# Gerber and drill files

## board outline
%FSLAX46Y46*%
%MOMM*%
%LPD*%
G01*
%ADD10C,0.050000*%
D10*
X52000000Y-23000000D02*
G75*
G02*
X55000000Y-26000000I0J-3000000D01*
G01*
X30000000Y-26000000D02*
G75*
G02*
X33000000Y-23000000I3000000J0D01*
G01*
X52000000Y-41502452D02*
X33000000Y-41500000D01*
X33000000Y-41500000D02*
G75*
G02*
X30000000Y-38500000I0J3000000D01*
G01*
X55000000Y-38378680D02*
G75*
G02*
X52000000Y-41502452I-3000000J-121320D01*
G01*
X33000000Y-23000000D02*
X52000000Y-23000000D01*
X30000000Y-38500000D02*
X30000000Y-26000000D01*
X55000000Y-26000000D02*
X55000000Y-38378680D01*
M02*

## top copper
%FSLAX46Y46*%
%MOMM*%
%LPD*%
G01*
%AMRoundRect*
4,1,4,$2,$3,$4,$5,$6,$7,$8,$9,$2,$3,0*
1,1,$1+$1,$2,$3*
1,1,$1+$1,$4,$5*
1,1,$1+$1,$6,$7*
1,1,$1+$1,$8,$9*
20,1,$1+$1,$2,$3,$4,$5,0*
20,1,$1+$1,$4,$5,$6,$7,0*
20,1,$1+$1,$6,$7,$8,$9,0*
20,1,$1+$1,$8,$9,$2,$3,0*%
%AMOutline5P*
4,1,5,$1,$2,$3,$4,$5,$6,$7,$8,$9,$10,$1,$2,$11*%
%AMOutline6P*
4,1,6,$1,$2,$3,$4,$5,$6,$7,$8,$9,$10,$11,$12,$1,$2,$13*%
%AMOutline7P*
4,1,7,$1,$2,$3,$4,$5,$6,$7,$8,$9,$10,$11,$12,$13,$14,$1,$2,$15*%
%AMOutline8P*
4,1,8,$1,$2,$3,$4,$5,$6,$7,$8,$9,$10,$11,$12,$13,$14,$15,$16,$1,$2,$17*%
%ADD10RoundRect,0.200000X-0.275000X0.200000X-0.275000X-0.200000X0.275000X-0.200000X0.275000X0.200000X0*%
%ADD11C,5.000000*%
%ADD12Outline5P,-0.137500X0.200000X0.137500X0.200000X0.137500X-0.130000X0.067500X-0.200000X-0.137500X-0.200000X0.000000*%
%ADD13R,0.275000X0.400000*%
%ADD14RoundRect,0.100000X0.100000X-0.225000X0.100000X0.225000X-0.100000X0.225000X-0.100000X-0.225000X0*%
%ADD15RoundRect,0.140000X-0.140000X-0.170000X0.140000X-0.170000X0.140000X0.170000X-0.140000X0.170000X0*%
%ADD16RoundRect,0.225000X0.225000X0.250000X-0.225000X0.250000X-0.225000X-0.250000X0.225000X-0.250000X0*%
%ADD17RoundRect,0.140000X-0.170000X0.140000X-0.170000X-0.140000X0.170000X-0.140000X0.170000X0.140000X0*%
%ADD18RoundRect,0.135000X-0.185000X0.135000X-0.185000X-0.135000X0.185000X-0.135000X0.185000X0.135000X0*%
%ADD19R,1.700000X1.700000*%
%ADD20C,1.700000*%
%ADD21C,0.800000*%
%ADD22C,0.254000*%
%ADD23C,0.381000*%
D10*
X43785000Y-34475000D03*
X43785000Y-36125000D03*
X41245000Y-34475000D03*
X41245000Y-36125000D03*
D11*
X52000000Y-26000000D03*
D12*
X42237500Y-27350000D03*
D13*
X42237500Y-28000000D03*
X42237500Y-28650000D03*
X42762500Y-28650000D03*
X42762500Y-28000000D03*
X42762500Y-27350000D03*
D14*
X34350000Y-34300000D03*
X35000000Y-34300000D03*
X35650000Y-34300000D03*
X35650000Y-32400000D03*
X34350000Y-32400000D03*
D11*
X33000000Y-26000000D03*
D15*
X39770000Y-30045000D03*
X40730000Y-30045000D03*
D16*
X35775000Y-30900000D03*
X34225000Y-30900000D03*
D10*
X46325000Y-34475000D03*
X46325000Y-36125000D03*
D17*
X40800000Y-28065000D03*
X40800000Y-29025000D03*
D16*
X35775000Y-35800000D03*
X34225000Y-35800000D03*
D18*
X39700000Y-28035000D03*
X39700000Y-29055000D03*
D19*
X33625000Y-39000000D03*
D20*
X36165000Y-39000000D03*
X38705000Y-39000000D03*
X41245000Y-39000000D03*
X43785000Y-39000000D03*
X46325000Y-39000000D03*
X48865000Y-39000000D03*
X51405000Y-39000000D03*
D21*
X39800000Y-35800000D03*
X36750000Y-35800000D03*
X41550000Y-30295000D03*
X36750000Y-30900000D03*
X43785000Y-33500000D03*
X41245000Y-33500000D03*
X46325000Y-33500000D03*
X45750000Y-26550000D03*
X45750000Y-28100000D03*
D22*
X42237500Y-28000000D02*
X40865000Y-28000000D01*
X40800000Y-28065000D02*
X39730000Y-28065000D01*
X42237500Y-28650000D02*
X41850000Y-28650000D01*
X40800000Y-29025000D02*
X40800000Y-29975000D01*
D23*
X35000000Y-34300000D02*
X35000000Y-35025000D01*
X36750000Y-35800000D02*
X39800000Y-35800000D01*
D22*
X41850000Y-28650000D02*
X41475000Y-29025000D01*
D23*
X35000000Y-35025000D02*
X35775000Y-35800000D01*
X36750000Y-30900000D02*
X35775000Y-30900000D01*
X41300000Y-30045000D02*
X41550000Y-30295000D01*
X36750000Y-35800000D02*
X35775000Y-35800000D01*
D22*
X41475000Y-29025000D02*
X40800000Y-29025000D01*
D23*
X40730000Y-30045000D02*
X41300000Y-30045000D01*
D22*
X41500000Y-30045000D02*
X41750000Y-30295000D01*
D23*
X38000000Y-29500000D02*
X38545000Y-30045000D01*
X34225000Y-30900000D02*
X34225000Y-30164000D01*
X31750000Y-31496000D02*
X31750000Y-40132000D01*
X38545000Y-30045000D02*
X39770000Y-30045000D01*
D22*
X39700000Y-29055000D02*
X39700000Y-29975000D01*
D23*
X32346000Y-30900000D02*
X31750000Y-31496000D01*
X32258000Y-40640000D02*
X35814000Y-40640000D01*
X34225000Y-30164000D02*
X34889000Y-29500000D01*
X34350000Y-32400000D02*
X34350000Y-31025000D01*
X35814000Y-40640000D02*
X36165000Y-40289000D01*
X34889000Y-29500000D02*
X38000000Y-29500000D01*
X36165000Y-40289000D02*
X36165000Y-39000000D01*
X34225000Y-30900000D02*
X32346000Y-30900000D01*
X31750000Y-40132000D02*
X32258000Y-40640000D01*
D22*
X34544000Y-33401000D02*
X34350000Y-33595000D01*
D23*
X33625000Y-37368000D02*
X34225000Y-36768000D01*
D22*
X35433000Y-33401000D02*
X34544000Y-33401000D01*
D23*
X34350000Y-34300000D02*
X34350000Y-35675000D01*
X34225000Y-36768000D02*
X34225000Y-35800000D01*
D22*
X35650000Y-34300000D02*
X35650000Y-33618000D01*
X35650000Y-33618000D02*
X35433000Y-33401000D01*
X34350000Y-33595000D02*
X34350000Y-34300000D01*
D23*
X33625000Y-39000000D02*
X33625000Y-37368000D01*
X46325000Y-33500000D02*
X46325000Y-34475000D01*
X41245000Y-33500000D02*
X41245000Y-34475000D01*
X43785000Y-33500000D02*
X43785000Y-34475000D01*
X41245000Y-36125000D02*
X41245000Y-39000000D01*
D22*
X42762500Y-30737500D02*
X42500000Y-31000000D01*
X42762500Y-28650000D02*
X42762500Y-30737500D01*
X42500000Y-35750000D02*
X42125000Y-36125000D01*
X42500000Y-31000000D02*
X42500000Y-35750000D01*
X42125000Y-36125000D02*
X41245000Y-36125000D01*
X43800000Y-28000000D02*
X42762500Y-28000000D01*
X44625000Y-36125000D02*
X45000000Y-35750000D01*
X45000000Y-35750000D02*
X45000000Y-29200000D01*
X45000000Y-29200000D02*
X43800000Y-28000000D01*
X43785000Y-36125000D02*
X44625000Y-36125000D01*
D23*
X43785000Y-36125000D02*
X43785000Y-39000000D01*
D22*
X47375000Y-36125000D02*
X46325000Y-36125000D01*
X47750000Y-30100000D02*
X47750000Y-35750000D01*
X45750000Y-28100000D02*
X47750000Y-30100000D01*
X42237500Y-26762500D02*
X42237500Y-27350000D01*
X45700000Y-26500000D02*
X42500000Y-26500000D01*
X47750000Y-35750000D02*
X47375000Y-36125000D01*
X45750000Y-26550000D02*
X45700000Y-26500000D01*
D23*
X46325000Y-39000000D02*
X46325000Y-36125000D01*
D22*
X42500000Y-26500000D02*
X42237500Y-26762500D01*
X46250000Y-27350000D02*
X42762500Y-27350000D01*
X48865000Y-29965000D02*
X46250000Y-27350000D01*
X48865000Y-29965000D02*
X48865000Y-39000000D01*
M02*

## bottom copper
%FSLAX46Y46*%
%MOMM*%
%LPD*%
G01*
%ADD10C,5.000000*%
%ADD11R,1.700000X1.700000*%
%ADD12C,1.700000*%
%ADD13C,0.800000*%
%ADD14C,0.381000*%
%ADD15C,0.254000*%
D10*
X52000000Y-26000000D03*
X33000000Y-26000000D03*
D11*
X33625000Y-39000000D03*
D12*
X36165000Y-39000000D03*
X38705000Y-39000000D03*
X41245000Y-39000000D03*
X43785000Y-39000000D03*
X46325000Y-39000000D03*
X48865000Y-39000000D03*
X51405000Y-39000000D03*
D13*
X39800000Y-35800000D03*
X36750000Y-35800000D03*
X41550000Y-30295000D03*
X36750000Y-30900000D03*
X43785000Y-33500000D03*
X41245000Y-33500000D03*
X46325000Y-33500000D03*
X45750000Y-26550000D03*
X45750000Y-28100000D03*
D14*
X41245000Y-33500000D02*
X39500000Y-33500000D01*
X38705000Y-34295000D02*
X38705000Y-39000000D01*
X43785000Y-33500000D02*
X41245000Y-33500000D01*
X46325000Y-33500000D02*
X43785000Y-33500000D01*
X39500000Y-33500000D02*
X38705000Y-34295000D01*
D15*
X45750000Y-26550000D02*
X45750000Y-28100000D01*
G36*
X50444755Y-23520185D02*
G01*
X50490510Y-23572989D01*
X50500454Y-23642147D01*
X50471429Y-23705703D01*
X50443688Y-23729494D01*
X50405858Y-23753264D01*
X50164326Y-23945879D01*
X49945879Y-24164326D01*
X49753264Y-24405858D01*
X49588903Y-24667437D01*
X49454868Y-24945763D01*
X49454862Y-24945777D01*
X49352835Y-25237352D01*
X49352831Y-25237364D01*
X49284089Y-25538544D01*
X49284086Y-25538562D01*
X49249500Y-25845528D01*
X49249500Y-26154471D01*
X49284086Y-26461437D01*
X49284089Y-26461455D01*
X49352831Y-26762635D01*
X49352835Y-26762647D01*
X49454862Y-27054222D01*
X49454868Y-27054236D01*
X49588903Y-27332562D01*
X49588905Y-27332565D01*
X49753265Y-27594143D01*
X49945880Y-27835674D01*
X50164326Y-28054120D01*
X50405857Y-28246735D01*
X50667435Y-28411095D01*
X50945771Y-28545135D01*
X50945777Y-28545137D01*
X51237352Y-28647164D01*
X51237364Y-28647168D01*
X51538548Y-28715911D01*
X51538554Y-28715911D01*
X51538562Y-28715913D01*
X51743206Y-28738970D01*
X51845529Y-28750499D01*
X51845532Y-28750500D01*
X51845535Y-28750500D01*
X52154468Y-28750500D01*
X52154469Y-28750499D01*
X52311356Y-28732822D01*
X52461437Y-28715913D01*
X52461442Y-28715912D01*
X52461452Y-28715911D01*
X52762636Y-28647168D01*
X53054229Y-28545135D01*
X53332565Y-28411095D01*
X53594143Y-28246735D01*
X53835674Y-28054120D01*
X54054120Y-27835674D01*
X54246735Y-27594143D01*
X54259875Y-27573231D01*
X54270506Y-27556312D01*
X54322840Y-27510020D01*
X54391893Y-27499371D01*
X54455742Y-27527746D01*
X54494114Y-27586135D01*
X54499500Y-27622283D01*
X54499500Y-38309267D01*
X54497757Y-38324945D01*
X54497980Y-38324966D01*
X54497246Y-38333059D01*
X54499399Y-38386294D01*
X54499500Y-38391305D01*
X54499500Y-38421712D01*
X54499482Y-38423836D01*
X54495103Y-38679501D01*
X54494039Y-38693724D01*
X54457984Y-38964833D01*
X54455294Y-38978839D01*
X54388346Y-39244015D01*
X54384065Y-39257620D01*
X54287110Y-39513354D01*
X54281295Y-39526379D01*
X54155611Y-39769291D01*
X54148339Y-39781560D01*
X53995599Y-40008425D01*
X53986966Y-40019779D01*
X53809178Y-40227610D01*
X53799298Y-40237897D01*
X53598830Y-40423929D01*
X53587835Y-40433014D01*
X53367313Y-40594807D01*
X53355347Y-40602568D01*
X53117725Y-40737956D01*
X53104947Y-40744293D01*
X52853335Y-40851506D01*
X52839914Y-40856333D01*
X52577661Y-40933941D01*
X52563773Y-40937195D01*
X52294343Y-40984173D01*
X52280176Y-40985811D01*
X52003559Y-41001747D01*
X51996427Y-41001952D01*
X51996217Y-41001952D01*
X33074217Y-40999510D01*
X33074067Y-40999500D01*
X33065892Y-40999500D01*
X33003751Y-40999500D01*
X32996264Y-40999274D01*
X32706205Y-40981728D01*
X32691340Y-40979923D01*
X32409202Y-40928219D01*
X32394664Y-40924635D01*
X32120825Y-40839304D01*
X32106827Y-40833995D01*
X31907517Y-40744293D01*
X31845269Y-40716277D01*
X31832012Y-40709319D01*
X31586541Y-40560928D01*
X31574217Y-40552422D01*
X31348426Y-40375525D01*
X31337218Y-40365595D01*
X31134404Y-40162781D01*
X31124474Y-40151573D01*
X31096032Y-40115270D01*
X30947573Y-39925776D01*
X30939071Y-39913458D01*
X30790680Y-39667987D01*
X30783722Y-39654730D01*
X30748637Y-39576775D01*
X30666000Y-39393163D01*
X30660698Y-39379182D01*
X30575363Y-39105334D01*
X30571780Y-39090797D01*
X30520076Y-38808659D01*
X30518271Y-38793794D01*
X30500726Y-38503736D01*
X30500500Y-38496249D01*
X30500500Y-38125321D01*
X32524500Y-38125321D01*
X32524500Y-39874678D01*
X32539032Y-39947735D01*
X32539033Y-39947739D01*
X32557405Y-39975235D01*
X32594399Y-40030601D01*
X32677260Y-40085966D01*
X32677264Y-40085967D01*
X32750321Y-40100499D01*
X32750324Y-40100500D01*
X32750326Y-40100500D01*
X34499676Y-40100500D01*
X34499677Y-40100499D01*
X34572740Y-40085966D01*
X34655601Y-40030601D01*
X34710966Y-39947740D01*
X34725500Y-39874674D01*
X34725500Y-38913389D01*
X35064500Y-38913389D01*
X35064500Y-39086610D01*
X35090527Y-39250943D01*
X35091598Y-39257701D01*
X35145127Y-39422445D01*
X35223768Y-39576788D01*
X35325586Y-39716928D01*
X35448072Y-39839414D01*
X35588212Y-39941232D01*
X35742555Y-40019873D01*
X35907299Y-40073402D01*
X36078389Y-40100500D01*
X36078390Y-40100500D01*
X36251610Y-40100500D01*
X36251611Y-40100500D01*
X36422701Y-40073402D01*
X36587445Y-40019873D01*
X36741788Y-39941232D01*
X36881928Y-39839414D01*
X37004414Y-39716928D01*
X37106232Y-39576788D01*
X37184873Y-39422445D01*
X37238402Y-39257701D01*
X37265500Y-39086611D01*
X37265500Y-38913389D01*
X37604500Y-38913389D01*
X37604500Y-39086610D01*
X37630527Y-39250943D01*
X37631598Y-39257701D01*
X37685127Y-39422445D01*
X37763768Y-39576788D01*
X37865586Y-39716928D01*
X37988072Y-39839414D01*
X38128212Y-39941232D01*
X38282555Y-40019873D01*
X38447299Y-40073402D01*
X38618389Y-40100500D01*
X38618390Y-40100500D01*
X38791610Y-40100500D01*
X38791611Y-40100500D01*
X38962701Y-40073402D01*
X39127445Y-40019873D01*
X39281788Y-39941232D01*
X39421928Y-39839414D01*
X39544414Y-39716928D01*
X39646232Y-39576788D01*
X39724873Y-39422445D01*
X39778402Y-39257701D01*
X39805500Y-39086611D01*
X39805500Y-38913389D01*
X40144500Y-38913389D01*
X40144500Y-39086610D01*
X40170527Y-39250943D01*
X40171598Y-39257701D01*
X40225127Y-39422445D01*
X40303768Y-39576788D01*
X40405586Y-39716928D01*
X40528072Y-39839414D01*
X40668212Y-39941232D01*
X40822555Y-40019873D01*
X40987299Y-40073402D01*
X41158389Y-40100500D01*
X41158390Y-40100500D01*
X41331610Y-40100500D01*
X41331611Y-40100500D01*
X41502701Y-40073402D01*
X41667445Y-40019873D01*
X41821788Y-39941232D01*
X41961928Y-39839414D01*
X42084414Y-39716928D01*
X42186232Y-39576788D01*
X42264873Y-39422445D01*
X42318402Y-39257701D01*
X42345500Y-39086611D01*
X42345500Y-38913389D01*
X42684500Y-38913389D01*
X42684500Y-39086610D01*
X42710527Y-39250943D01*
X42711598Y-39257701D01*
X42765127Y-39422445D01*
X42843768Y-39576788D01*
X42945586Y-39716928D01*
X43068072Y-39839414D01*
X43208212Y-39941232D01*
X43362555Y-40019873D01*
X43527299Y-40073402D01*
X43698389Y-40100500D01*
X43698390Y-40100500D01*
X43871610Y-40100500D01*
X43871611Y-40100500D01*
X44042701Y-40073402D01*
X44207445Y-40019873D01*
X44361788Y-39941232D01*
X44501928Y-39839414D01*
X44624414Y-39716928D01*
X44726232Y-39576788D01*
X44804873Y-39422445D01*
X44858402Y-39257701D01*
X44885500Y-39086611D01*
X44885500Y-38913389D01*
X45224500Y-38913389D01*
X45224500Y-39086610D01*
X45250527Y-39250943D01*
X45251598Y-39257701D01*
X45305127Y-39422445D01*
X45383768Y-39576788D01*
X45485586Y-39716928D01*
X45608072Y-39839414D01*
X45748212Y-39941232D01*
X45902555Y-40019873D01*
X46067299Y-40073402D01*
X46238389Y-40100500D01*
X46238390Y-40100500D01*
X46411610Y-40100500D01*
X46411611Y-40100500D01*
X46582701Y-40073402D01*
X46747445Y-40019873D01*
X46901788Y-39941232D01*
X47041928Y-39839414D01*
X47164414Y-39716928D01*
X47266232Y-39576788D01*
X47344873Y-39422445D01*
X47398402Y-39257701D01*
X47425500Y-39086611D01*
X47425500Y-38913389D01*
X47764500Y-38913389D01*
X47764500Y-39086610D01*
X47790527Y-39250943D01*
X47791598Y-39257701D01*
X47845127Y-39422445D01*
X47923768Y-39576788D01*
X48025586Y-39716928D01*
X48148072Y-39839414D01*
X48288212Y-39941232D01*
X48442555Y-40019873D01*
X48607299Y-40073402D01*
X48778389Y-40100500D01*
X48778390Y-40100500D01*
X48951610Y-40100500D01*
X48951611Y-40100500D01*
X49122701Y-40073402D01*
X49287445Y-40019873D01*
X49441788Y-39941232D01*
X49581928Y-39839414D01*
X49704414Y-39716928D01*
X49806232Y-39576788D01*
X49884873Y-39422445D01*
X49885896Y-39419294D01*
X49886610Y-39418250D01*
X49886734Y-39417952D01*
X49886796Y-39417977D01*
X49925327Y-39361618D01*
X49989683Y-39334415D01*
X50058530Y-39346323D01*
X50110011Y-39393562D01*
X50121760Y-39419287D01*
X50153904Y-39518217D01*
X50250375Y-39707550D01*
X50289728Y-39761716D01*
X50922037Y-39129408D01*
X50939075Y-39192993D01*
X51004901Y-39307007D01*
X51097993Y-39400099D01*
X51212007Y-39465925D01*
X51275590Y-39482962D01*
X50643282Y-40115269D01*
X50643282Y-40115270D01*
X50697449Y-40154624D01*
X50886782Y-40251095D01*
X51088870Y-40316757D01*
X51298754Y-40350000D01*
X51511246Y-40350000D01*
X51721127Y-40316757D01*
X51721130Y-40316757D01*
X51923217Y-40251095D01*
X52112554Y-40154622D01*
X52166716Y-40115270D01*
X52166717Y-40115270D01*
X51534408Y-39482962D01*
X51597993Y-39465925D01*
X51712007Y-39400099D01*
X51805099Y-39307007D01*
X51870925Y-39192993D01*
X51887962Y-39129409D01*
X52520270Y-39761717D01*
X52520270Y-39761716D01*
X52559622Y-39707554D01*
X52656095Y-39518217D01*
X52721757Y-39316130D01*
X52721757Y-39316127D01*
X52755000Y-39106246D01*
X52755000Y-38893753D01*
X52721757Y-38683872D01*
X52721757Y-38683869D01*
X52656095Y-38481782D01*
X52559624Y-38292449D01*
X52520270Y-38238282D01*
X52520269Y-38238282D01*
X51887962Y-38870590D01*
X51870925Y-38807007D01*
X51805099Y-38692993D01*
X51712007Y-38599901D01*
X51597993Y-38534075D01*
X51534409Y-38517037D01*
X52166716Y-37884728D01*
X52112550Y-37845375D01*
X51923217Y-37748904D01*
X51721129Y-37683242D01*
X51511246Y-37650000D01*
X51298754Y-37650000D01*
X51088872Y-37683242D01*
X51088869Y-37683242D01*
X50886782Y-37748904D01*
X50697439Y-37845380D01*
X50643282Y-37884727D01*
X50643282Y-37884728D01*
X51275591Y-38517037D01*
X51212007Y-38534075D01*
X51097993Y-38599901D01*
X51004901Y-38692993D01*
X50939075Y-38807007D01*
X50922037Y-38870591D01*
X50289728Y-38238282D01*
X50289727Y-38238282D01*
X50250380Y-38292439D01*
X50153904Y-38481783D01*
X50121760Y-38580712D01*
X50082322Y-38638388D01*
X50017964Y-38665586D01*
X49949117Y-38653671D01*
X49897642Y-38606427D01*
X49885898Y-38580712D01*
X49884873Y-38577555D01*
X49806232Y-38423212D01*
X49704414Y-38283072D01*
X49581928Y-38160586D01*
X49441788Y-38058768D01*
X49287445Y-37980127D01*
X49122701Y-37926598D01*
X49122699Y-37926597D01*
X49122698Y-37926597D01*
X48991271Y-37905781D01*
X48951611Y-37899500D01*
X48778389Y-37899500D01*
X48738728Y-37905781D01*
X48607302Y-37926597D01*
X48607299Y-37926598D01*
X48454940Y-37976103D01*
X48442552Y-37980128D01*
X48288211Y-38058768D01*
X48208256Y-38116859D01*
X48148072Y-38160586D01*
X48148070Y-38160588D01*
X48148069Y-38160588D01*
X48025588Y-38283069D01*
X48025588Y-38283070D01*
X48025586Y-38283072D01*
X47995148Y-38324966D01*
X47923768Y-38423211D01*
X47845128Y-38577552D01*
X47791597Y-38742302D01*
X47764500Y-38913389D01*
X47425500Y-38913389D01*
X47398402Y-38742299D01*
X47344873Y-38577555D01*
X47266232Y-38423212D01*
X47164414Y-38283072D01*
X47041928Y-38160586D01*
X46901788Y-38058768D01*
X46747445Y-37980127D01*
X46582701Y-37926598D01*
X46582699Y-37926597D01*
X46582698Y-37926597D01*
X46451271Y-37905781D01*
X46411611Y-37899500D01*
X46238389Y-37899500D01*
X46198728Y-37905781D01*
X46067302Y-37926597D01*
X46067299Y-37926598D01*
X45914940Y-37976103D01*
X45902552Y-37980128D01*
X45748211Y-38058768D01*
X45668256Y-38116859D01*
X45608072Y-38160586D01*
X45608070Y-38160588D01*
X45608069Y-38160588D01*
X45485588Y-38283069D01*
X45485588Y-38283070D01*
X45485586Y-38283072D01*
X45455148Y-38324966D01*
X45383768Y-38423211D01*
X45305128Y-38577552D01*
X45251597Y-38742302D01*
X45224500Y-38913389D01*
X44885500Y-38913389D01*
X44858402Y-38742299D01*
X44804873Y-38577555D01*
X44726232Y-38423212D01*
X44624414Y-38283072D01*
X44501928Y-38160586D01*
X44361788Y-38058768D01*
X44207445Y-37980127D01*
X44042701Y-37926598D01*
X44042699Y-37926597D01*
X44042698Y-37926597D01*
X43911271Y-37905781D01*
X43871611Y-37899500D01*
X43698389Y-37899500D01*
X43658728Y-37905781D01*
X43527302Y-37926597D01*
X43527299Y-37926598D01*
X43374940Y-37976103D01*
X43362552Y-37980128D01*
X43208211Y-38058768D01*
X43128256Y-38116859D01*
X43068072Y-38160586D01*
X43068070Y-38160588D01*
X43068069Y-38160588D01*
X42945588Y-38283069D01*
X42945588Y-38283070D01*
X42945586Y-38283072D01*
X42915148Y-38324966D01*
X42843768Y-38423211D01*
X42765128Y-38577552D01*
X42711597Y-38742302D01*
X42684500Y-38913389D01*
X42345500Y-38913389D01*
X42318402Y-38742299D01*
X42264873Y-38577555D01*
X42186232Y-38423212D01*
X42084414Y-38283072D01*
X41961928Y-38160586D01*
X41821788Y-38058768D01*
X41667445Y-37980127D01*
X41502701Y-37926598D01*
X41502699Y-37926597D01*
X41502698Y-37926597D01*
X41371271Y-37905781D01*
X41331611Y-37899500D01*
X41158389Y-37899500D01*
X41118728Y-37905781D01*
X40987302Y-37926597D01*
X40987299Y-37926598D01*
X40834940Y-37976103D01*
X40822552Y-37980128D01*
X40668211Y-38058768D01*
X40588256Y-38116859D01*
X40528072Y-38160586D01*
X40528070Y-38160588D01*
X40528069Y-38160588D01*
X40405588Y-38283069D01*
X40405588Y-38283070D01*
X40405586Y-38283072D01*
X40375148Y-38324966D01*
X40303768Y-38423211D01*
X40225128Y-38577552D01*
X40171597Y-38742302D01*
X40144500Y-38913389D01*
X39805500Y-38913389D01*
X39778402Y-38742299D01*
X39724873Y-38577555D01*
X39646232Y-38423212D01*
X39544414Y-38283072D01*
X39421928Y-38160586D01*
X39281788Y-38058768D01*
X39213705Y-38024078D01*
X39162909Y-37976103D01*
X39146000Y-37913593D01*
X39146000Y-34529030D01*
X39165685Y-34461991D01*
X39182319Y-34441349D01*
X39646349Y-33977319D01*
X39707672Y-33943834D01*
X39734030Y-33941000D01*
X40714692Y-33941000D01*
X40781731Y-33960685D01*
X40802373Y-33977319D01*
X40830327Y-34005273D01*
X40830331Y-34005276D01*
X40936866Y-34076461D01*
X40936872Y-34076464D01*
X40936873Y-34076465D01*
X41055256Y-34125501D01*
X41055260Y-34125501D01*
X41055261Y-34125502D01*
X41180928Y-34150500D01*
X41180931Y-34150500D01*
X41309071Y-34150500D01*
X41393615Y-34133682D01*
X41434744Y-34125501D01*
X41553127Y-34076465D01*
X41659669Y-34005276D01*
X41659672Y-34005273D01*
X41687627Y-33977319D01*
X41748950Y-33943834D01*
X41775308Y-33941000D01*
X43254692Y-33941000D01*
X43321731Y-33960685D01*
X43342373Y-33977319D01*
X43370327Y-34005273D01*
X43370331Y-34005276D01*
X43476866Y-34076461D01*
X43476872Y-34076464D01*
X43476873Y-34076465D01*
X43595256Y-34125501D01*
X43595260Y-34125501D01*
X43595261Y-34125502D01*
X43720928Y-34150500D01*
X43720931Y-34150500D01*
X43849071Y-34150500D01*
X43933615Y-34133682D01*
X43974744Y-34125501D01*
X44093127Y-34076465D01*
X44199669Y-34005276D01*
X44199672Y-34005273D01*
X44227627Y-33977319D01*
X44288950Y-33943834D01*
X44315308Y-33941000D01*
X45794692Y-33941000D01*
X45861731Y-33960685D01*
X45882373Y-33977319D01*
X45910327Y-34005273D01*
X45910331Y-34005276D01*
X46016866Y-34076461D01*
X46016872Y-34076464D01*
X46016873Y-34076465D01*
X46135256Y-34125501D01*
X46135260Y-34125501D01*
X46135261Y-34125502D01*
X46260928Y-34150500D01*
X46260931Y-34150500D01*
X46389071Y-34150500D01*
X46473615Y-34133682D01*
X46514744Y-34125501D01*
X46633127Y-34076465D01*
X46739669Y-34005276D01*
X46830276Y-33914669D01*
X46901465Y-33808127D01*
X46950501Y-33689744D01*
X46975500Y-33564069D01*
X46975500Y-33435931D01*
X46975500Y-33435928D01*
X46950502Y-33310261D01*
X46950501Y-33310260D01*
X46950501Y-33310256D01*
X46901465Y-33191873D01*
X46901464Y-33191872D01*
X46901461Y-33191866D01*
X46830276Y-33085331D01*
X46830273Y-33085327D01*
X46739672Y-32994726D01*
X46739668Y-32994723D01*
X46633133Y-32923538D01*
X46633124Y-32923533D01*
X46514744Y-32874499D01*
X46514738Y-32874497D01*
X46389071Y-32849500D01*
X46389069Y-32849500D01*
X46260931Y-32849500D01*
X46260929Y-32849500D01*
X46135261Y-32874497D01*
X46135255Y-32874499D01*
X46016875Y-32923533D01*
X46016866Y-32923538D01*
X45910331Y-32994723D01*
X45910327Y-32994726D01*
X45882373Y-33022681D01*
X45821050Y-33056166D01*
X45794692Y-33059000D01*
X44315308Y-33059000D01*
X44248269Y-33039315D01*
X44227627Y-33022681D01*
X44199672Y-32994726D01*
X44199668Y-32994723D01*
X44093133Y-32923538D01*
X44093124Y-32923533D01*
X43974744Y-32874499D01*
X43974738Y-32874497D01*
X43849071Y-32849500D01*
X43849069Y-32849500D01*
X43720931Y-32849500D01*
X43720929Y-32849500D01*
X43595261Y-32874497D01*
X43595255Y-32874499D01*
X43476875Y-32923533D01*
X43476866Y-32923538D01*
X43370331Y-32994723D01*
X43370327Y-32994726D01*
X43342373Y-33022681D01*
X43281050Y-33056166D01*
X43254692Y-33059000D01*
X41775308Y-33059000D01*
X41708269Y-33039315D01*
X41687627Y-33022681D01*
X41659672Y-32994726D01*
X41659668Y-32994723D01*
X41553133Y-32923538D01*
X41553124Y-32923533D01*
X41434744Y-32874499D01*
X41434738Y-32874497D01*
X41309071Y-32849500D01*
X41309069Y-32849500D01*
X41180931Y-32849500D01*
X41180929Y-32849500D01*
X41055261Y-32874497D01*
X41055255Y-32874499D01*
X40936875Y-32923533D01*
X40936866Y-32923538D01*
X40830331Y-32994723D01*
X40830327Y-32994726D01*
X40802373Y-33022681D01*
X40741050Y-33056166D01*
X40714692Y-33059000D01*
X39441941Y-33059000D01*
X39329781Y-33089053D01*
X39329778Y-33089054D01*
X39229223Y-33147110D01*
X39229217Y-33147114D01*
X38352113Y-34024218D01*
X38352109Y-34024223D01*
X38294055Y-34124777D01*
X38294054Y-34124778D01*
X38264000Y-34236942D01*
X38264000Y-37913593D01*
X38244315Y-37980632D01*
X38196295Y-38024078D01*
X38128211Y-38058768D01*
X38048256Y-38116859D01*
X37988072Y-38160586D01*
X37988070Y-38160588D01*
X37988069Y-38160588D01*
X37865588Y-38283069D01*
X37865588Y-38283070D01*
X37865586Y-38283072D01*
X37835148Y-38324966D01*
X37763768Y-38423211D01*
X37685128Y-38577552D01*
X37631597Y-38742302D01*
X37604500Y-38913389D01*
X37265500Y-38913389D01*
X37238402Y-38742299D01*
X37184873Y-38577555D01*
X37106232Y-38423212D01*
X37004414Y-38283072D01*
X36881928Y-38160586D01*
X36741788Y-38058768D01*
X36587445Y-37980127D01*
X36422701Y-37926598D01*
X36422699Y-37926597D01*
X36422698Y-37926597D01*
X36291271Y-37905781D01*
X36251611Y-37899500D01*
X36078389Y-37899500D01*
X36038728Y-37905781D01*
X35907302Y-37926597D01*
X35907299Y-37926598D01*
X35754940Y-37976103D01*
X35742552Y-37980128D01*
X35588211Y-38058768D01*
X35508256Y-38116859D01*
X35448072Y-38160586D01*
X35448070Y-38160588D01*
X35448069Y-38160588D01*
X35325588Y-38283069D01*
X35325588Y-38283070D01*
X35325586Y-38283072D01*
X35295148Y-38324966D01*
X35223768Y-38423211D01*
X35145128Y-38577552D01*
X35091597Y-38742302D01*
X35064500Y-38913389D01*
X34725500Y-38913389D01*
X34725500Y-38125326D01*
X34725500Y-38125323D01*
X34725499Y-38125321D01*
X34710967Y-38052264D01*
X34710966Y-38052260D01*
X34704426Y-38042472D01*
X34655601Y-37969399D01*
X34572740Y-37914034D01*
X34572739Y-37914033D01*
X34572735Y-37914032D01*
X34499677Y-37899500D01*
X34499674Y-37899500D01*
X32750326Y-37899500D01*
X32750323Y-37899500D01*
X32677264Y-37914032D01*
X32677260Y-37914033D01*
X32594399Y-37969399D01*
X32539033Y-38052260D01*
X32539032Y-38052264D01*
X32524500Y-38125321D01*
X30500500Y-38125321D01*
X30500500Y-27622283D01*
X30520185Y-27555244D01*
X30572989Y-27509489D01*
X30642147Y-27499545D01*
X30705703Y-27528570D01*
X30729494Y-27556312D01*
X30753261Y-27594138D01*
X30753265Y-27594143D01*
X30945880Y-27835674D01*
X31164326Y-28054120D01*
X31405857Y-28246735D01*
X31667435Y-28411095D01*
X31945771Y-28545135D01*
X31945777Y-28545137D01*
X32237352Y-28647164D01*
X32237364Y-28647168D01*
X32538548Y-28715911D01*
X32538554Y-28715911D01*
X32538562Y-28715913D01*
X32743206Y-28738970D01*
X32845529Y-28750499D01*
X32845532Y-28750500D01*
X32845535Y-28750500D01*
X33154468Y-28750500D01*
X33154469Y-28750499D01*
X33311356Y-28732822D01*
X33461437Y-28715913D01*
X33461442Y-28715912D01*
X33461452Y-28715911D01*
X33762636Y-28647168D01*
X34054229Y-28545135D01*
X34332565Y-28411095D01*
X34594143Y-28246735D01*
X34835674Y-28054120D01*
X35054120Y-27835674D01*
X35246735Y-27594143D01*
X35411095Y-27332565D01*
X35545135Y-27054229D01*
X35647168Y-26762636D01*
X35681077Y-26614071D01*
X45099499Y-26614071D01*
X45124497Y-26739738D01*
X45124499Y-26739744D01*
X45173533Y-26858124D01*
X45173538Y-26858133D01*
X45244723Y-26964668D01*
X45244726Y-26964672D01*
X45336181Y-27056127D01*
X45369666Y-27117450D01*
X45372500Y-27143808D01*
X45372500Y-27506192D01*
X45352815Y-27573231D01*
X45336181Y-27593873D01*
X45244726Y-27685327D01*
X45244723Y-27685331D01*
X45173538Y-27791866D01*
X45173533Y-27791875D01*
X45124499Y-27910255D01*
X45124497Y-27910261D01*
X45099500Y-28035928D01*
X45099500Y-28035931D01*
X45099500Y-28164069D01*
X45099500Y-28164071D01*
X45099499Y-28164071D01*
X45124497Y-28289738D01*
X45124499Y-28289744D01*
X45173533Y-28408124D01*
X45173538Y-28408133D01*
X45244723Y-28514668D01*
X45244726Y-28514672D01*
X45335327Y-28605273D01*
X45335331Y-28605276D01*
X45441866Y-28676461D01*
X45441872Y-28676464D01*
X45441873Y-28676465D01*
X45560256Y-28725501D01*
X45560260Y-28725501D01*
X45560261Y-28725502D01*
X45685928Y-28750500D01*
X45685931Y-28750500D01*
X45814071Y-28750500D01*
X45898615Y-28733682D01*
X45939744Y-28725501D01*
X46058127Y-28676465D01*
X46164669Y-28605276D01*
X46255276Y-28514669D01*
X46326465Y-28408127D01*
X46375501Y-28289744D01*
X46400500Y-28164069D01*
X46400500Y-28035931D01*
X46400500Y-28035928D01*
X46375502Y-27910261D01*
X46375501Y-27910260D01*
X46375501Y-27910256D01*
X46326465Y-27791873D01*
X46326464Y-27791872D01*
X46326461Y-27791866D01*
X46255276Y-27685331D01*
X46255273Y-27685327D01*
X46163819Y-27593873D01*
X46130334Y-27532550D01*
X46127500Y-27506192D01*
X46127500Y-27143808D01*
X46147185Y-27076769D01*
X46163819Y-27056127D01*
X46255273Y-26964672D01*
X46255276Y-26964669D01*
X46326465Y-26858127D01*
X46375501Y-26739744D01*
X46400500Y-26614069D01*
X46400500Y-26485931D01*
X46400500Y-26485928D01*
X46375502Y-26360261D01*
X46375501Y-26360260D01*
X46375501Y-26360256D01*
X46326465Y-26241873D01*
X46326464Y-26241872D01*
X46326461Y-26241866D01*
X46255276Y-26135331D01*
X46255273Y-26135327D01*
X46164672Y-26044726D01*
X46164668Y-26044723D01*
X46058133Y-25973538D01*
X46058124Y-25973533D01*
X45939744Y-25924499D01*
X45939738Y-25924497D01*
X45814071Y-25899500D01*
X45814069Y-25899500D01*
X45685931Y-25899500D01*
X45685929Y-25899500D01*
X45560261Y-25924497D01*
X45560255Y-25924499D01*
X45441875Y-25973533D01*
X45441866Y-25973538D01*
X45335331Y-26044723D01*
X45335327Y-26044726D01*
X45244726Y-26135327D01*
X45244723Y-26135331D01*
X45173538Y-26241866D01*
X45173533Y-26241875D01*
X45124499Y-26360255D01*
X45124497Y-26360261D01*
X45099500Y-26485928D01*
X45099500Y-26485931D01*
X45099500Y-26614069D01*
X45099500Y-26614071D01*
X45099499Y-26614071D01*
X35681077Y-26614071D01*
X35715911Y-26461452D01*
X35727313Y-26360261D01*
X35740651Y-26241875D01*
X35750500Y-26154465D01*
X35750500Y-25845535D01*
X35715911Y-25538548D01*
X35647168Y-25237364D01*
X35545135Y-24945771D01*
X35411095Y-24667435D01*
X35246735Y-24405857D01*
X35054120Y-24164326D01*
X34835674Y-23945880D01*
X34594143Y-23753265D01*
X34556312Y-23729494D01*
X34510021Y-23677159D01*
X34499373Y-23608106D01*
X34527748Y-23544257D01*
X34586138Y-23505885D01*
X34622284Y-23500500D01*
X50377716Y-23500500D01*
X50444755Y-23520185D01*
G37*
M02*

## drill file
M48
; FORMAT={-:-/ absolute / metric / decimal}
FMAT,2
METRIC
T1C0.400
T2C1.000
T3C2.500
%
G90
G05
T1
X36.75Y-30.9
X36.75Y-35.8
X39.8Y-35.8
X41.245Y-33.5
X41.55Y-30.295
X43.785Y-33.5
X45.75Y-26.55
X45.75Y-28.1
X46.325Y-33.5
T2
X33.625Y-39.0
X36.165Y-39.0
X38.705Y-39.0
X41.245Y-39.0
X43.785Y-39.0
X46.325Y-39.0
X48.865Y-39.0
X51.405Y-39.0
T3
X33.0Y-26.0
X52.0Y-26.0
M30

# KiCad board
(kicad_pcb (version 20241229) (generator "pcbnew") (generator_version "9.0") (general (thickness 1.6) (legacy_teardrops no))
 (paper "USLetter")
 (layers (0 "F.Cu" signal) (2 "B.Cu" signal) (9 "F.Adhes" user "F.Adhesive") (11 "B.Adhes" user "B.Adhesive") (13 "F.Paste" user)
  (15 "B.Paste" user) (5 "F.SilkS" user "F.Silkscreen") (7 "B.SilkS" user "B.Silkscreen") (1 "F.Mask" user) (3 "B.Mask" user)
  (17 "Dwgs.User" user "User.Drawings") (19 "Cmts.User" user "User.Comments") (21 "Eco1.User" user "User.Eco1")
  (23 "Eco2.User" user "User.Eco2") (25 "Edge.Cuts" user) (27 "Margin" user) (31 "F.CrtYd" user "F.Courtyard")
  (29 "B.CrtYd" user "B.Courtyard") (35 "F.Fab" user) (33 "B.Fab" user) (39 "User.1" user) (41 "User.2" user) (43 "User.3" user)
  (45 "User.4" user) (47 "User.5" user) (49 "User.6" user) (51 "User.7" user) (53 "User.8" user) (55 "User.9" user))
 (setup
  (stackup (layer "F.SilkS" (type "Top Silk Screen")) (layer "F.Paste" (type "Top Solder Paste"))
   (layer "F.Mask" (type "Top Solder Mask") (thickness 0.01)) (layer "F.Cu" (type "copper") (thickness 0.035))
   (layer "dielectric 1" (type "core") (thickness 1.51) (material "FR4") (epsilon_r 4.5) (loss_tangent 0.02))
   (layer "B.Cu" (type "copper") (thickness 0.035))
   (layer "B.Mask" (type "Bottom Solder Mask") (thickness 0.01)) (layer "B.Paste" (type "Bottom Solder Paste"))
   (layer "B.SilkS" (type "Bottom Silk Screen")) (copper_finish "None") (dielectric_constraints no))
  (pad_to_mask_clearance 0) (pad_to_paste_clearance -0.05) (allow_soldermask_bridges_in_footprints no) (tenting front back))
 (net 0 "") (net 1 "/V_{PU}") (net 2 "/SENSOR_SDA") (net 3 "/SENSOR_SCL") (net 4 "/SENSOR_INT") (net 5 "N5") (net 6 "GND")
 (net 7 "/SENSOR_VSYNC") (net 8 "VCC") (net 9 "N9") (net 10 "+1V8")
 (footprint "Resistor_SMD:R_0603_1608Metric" (layer "F.Cu") (at 43.785 35.3 -90)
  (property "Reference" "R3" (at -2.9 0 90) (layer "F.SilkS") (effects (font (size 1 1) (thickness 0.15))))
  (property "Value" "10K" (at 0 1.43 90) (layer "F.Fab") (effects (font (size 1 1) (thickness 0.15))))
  (pad "1" smd roundrect (at -0.825 0 270) (size 0.8 0.95) (layers "F.Cu" "F.Mask" "F.Paste") (roundrect_rratio 0.25) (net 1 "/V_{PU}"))
  (pad "2" smd roundrect (at 0.825 0 270) (size 0.8 0.95) (layers "F.Cu" "F.Mask" "F.Paste") (roundrect_rratio 0.25) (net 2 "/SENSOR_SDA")))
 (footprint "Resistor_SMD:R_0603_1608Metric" (layer "F.Cu") (at 41.245 35.3 -90)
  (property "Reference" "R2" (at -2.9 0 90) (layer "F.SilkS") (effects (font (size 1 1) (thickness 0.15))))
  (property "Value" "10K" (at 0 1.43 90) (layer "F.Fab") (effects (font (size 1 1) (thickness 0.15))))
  (pad "1" smd roundrect (at -0.825 0 270) (size 0.8 0.95) (layers "F.Cu" "F.Mask" "F.Paste") (roundrect_rratio 0.25) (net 1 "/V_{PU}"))
  (pad "2" smd roundrect (at 0.825 0 270) (size 0.8 0.95) (layers "F.Cu" "F.Mask" "F.Paste") (roundrect_rratio 0.25) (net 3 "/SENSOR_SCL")))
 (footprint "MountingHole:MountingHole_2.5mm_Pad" (layer "F.Cu") (at 52 26)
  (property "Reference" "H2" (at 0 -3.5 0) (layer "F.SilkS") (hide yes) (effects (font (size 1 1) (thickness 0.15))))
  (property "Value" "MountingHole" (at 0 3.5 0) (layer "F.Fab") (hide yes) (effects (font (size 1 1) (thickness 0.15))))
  (pad "1" thru_hole circle (at 0 0) (size 5 5) (drill 2.5) (layers "*.Cu" "*.Mask") (remove_unused_layers no)))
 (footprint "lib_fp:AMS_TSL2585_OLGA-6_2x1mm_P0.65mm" (layer "F.Cu") (at 42.5 28)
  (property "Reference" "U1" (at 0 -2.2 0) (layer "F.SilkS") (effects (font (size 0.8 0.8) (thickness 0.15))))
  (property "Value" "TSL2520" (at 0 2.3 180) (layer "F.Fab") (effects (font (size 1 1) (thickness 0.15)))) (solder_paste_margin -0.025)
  (pad "1" smd roundrect (at -0.2625 -0.65) (size 0.275 0.4) (layers "F.Cu" "F.Mask" "F.Paste") (roundrect_rratio 0)
   (chamfer_ratio 0.254545) (chamfer bottom_right) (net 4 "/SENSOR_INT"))
  (pad "2" smd rect (at -0.2625 0) (size 0.275 0.4) (layers "F.Cu" "F.Mask" "F.Paste") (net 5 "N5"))
  (pad "3" smd rect (at -0.2625 0.65) (size 0.275 0.4) (layers "F.Cu" "F.Mask" "F.Paste") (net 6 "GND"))
  (pad "4" smd rect (at 0.2625 0.65) (size 0.275 0.4) (layers "F.Cu" "F.Mask" "F.Paste") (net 3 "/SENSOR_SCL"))
  (pad "5" smd rect (at 0.2625 0) (size 0.275 0.4) (layers "F.Cu" "F.Mask" "F.Paste") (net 2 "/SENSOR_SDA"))
  (pad "6" smd rect (at 0.2625 -0.65) (size 0.275 0.4) (layers "F.Cu" "F.Mask" "F.Paste") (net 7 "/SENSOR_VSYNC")))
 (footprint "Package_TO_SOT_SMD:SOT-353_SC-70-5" (layer "F.Cu") (at 35 33.35 90)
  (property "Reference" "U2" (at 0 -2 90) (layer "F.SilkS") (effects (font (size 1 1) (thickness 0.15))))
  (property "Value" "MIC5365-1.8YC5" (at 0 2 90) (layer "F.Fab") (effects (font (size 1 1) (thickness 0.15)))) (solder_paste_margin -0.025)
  (pad "1" smd roundrect (at -0.95 -0.65 90) (size 0.65 0.4) (layers "F.Cu" "F.Mask" "F.Paste") (roundrect_rratio 0.25) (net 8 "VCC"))
  (pad "2" smd roundrect (at -0.95 0 90) (size 0.65 0.4) (layers "F.Cu" "F.Mask" "F.Paste") (roundrect_rratio 0.25) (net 6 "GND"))
  (pad "3" smd roundrect (at -0.95 0.65 90) (size 0.65 0.4) (layers "F.Cu" "F.Mask" "F.Paste") (roundrect_rratio 0.25) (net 8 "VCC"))
  (pad "4" smd roundrect (at 0.95 0.65 90) (size 0.65 0.4) (layers "F.Cu" "F.Mask" "F.Paste") (roundrect_rratio 0.25) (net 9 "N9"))
  (pad "5" smd roundrect (at 0.95 -0.65 90) (size 0.65 0.4) (layers "F.Cu" "F.Mask" "F.Paste") (roundrect_rratio 0.25) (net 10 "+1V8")))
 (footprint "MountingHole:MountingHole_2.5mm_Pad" (layer "F.Cu") (at 33 26)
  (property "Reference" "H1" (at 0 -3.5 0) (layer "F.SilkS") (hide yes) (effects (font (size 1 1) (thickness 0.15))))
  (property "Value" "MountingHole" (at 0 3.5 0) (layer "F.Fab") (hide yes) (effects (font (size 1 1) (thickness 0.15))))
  (pad "1" thru_hole circle (at 0 0) (size 5 5) (drill 2.5) (layers "*.Cu" "*.Mask") (remove_unused_layers no)))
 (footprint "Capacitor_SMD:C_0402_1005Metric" (layer "F.Cu") (at 40.25 30.045)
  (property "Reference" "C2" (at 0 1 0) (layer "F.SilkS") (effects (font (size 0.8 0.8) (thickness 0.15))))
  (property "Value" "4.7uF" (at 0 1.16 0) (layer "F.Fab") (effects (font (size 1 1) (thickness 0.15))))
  (pad "1" smd roundrect (at -0.48 0) (size 0.56 0.62) (layers "F.Cu" "F.Mask" "F.Paste") (roundrect_rratio 0.25) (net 10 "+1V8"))
  (pad "2" smd roundrect (at 0.48 0) (size 0.56 0.62) (layers "F.Cu" "F.Mask" "F.Paste") (roundrect_rratio 0.25) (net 6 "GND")))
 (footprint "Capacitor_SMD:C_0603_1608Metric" (layer "F.Cu") (at 35 30.9 180)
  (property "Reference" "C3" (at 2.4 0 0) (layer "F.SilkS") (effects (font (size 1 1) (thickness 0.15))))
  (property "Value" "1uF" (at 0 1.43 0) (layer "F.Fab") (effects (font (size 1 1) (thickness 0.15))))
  (pad "1" smd roundrect (at -0.775 0 180) (size 0.9 0.95) (layers "F.Cu" "F.Mask" "F.Paste") (roundrect_rratio 0.25) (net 6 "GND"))
  (pad "2" smd roundrect (at 0.775 0 180) (size 0.9 0.95) (layers "F.Cu" "F.Mask" "F.Paste") (roundrect_rratio 0.25) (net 10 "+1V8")))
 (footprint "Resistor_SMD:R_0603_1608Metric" (layer "F.Cu") (at 46.325 35.3 -90)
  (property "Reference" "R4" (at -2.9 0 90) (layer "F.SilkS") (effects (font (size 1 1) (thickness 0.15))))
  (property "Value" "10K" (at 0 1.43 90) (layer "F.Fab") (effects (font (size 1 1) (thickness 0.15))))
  (pad "1" smd roundrect (at -0.825 0 270) (size 0.8 0.95) (layers "F.Cu" "F.Mask" "F.Paste") (roundrect_rratio 0.25) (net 1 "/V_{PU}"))
  (pad "2" smd roundrect (at 0.825 0 270) (size 0.8 0.95) (layers "F.Cu" "F.Mask" "F.Paste") (roundrect_rratio 0.25) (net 4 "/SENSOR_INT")))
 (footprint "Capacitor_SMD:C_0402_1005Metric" (layer "F.Cu") (at 40.8 28.545 -90)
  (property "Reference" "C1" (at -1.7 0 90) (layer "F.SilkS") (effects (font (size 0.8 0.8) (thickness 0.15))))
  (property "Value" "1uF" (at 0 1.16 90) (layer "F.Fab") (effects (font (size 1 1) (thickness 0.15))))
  (pad "1" smd roundrect (at -0.48 0 270) (size 0.56 0.62) (layers "F.Cu" "F.Mask" "F.Paste") (roundrect_rratio 0.25) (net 5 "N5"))
  (pad "2" smd roundrect (at 0.48 0 270) (size 0.56 0.62) (layers "F.Cu" "F.Mask" "F.Paste") (roundrect_rratio 0.25) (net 6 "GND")))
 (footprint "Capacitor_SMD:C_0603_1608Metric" (layer "F.Cu") (at 35 35.8 180)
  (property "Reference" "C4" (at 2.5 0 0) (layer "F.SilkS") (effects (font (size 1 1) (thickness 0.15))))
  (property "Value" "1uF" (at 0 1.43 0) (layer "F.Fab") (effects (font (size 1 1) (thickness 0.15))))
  (pad "1" smd roundrect (at -0.775 0 180) (size 0.9 0.95) (layers "F.Cu" "F.Mask" "F.Paste") (roundrect_rratio 0.25) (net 6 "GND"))
  (pad "2" smd roundrect (at 0.775 0 180) (size 0.9 0.95) (layers "F.Cu" "F.Mask" "F.Paste") (roundrect_rratio 0.25) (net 8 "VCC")))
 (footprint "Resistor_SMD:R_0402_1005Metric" (layer "F.Cu") (at 39.7 28.545 -90)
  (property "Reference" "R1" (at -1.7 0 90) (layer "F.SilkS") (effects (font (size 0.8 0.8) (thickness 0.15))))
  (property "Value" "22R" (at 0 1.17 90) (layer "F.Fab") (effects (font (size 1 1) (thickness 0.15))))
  (pad "1" smd roundrect (at -0.51 0 270) (size 0.54 0.64) (layers "F.Cu" "F.Mask" "F.Paste") (roundrect_rratio 0.25) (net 5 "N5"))
  (pad "2" smd roundrect (at 0.51 0 270) (size 0.54 0.64) (layers "F.Cu" "F.Mask" "F.Paste") (roundrect_rratio 0.25) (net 10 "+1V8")))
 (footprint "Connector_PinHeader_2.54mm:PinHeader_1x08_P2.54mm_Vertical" (layer "B.Cu") (at 33.625 39 -90)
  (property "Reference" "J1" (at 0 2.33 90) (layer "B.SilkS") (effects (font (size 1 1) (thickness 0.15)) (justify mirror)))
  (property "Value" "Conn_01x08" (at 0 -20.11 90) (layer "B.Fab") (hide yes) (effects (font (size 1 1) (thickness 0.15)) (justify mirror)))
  (pad "1" thru_hole rect (at 0 0 270) (size 1.7 1.7) (drill 1) (layers "*.Cu" "*.Mask") (remove_unused_layers no) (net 8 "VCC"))
  (pad "2" thru_hole circle (at 0 -2.54 270) (size 1.7 1.7) (drill 1) (layers "*.Cu" "*.Mask") (remove_unused_layers no) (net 10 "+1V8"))
  (pad "3" thru_hole circle (at 0 -5.08 270) (size 1.7 1.7) (drill 1) (layers "*.Cu" "*.Mask") (remove_unused_layers no) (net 1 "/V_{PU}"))
  (pad "4" thru_hole circle (at 0 -7.62 270) (size 1.7 1.7) (drill 1) (layers "*.Cu" "*.Mask") (remove_unused_layers no)
   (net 3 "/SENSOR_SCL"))
  (pad "5" thru_hole circle (at 0 -10.16 270) (size 1.7 1.7) (drill 1) (layers "*.Cu" "*.Mask") (remove_unused_layers no)
   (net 2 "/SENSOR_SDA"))
  (pad "6" thru_hole circle (at 0 -12.7 270) (size 1.7 1.7) (drill 1) (layers "*.Cu" "*.Mask") (remove_unused_layers no)
   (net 4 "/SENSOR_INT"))
  (pad "7" thru_hole circle (at 0 -15.24 270) (size 1.7 1.7) (drill 1) (layers "*.Cu" "*.Mask") (remove_unused_layers no)
   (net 7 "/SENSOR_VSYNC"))
  (pad "8" thru_hole circle (at 0 -17.78 270) (size 1.7 1.7) (drill 1) (layers "*.Cu" "*.Mask") (remove_unused_layers no) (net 6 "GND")))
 (gr_arc (start 52 23) (mid 54.12132 23.87868) (end 55 26) (stroke (width 0.05) (type default)) (layer "Edge.Cuts"))
 (gr_arc (start 30 26) (mid 30.87868 23.87868) (end 33 23) (stroke (width 0.05) (type default)) (layer "Edge.Cuts"))
 (gr_line (start 52 41.502452) (end 33 41.5) (stroke (width 0.05) (type default)) (layer "Edge.Cuts"))
 (gr_arc (start 33 41.5) (mid 30.87868 40.62132) (end 30 38.5) (stroke (width 0.05) (type default)) (layer "Edge.Cuts"))
 (gr_arc (start 55 38.37868) (mid 54.165523 40.579719) (end 52 41.502452) (stroke (width 0.05) (type default)) (layer "Edge.Cuts"))
 (gr_line (start 33 23) (end 52 23) (stroke (width 0.05) (type default)) (layer "Edge.Cuts"))
 (gr_line (start 30 38.5) (end 30 26) (stroke (width 0.05) (type default)) (layer "Edge.Cuts"))
 (gr_line (start 55 26) (end 55 38.37868) (stroke (width 0.05) (type default)) (layer "Edge.Cuts"))
 (segment (start 42.2375 28) (end 40.865 28) (width 0.254) (layer "F.Cu") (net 5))
 (segment (start 40.8 28.065) (end 39.73 28.065) (width 0.254) (layer "F.Cu") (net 5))
 (segment (start 42.2375 28.65) (end 41.85 28.65) (width 0.254) (layer "F.Cu") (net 6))
 (segment (start 40.8 29.025) (end 40.8 29.975) (width 0.254) (layer "F.Cu") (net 6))
 (segment (start 35 34.3) (end 35 35.025) (width 0.381) (layer "F.Cu") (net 6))
 (segment (start 36.75 35.8) (end 39.8 35.8) (width 0.381) (layer "F.Cu") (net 6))
 (segment (start 41.85 28.65) (end 41.475 29.025) (width 0.254) (layer "F.Cu") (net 6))
 (segment (start 35 35.025) (end 35.775 35.8) (width 0.381) (layer "F.Cu") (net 6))
 (segment (start 36.75 30.9) (end 35.775 30.9) (width 0.381) (layer "F.Cu") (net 6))
 (segment (start 41.3 30.045) (end 41.55 30.295) (width 0.381) (layer "F.Cu") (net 6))
 (segment (start 36.75 35.8) (end 35.775 35.8) (width 0.381) (layer "F.Cu") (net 6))
 (segment (start 41.475 29.025) (end 40.8 29.025) (width 0.254) (layer "F.Cu") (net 6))
 (segment (start 40.73 30.045) (end 41.3 30.045) (width 0.381) (layer "F.Cu") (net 6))
 (segment (start 41.5 30.045) (end 41.75 30.295) (width 0.254) (layer "F.Cu") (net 6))
 (via (at 39.8 35.8) (size 0.8) (drill 0.4) (layers "F.Cu" "B.Cu") (free yes) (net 6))
 (via (at 36.75 35.8) (size 0.8) (drill 0.4) (layers "F.Cu" "B.Cu") (free yes) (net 6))
 (via (at 41.55 30.295) (size 0.8) (drill 0.4) (layers "F.Cu" "B.Cu") (free yes) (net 6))
 (via (at 36.75 30.9) (size 0.8) (drill 0.4) (layers "F.Cu" "B.Cu") (free yes) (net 6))
 (segment (start 38 29.5) (end 38.545 30.045) (width 0.381) (layer "F.Cu") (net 10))
 (segment (start 34.225 30.9) (end 34.225 30.164) (width 0.381) (layer "F.Cu") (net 10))
 (segment (start 31.75 31.496) (end 31.75 40.132) (width 0.381) (layer "F.Cu") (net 10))
 (segment (start 38.545 30.045) (end 39.77 30.045) (width 0.381) (layer "F.Cu") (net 10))
 (segment (start 39.7 29.055) (end 39.7 29.975) (width 0.254) (layer "F.Cu") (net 10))
 (segment (start 32.346 30.9) (end 31.75 31.496) (width 0.381) (layer "F.Cu") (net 10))
 (segment (start 32.258 40.64) (end 35.814 40.64) (width 0.381) (layer "F.Cu") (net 10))
 (segment (start 34.225 30.164) (end 34.889 29.5) (width 0.381) (layer "F.Cu") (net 10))
 (segment (start 34.35 32.4) (end 34.35 31.025) (width 0.381) (layer "F.Cu") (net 10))
 (segment (start 35.814 40.64) (end 36.165 40.289) (width 0.381) (layer "F.Cu") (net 10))
 (segment (start 34.889 29.5) (end 38 29.5) (width 0.381) (layer "F.Cu") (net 10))
 (segment (start 36.165 40.289) (end 36.165 39) (width 0.381) (layer "F.Cu") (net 10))
 (segment (start 34.225 30.9) (end 32.346 30.9) (width 0.381) (layer "F.Cu") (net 10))
 (segment (start 31.75 40.132) (end 32.258 40.64) (width 0.381) (layer "F.Cu") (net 10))
 (segment (start 34.544 33.401) (end 34.35 33.595) (width 0.254) (layer "F.Cu") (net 8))
 (segment (start 33.625 37.368) (end 34.225 36.768) (width 0.381) (layer "F.Cu") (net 8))
 (segment (start 35.433 33.401) (end 34.544 33.401) (width 0.254) (layer "F.Cu") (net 8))
 (segment (start 34.35 34.3) (end 34.35 35.675) (width 0.381) (layer "F.Cu") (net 8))
 (segment (start 34.225 36.768) (end 34.225 35.8) (width 0.381) (layer "F.Cu") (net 8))
 (segment (start 35.65 34.3) (end 35.65 33.618) (width 0.254) (layer "F.Cu") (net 8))
 (segment (start 35.65 33.618) (end 35.433 33.401) (width 0.254) (layer "F.Cu") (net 8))
 (segment (start 34.35 33.595) (end 34.35 34.3) (width 0.254) (layer "F.Cu") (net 8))
 (segment (start 33.625 39) (end 33.625 37.368) (width 0.381) (layer "F.Cu") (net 8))
 (segment (start 46.325 33.5) (end 46.325 34.475) (width 0.381) (layer "F.Cu") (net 1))
 (segment (start 41.245 33.5) (end 41.245 34.475) (width 0.381) (layer "F.Cu") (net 1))
 (segment (start 43.785 33.5) (end 43.785 34.475) (width 0.381) (layer "F.Cu") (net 1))
 (via (at 43.785 33.5) (size 0.8) (drill 0.4) (layers "F.Cu" "B.Cu") (free yes) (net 1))
 (via (at 41.245 33.5) (size 0.8) (drill 0.4) (layers "F.Cu" "B.Cu") (free yes) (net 1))
 (via (at 46.325 33.5) (size 0.8) (drill 0.4) (layers "F.Cu" "B.Cu") (free yes) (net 1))
 (segment (start 41.245 33.5) (end 39.5 33.5) (width 0.381) (layer "B.Cu") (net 1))
 (segment (start 38.705 34.295) (end 38.705 39) (width 0.381) (layer "B.Cu") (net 1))
 (segment (start 43.785 33.5) (end 41.245 33.5) (width 0.381) (layer "B.Cu") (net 1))
 (segment (start 46.325 33.5) (end 43.785 33.5) (width 0.381) (layer "B.Cu") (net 1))
 (segment (start 39.5 33.5) (end 38.705 34.295) (width 0.381) (layer "B.Cu") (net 1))
 (segment (start 41.245 36.125) (end 41.245 39) (width 0.381) (layer "F.Cu") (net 3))
 (segment (start 42.7625 30.7375) (end 42.5 31) (width 0.254) (layer "F.Cu") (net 3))
 (segment (start 42.7625 28.65) (end 42.7625 30.7375) (width 0.254) (layer "F.Cu") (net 3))
 (segment (start 42.5 35.75) (end 42.125 36.125) (width 0.254) (layer "F.Cu") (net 3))
 (segment (start 42.5 31) (end 42.5 35.75) (width 0.254) (layer "F.Cu") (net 3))
 (segment (start 42.125 36.125) (end 41.245 36.125) (width 0.254) (layer "F.Cu") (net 3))
 (segment (start 43.8 28) (end 42.7625 28) (width 0.254) (layer "F.Cu") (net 2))
 (segment (start 44.625 36.125) (end 45 35.75) (width 0.254) (layer "F.Cu") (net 2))
 (segment (start 45 35.75) (end 45 29.2) (width 0.254) (layer "F.Cu") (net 2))
 (segment (start 45 29.2) (end 43.8 28) (width 0.254) (layer "F.Cu") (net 2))
 (segment (start 43.785 36.125) (end 44.625 36.125) (width 0.254) (layer "F.Cu") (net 2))
 (segment (start 43.785 36.125) (end 43.785 39) (width 0.381) (layer "F.Cu") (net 2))
 (segment (start 47.375 36.125) (end 46.325 36.125) (width 0.254) (layer "F.Cu") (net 4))
 (segment (start 47.75 30.1) (end 47.75 35.75) (width 0.254) (layer "F.Cu") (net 4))
 (segment (start 45.75 28.1) (end 47.75 30.1) (width 0.254) (layer "F.Cu") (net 4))
 (segment (start 42.2375 26.7625) (end 42.2375 27.35) (width 0.254) (layer "F.Cu") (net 4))
 (segment (start 45.7 26.5) (end 42.5 26.5) (width 0.254) (layer "F.Cu") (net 4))
 (segment (start 47.75 35.75) (end 47.375 36.125) (width 0.254) (layer "F.Cu") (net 4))
 (segment (start 45.75 26.55) (end 45.7 26.5) (width 0.254) (layer "F.Cu") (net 4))
 (segment (start 46.325 39) (end 46.325 36.125) (width 0.381) (layer "F.Cu") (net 4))
 (segment (start 42.5 26.5) (end 42.2375 26.7625) (width 0.254) (layer "F.Cu") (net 4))
 (via (at 45.75 26.55) (size 0.8) (drill 0.4) (layers "F.Cu" "B.Cu") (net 4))
 (via (at 45.75 28.1) (size 0.8) (drill 0.4) (layers "F.Cu" "B.Cu") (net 4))
 (segment (start 45.75 26.55) (end 45.75 28.1) (width 0.254) (layer "B.Cu") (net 4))
 (segment (start 46.25 27.35) (end 42.7625 27.35) (width 0.254) (layer "F.Cu") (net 7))
 (segment (start 48.865 29.965) (end 46.25 27.35) (width 0.254) (layer "F.Cu") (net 7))
 (segment (start 48.865 29.965) (end 48.865 39) (width 0.254) (layer "F.Cu") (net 7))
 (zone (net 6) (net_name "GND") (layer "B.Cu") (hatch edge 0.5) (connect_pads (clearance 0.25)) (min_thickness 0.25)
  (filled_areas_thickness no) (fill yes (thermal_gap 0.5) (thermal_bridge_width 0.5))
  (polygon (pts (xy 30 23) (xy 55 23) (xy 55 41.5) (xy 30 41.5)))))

